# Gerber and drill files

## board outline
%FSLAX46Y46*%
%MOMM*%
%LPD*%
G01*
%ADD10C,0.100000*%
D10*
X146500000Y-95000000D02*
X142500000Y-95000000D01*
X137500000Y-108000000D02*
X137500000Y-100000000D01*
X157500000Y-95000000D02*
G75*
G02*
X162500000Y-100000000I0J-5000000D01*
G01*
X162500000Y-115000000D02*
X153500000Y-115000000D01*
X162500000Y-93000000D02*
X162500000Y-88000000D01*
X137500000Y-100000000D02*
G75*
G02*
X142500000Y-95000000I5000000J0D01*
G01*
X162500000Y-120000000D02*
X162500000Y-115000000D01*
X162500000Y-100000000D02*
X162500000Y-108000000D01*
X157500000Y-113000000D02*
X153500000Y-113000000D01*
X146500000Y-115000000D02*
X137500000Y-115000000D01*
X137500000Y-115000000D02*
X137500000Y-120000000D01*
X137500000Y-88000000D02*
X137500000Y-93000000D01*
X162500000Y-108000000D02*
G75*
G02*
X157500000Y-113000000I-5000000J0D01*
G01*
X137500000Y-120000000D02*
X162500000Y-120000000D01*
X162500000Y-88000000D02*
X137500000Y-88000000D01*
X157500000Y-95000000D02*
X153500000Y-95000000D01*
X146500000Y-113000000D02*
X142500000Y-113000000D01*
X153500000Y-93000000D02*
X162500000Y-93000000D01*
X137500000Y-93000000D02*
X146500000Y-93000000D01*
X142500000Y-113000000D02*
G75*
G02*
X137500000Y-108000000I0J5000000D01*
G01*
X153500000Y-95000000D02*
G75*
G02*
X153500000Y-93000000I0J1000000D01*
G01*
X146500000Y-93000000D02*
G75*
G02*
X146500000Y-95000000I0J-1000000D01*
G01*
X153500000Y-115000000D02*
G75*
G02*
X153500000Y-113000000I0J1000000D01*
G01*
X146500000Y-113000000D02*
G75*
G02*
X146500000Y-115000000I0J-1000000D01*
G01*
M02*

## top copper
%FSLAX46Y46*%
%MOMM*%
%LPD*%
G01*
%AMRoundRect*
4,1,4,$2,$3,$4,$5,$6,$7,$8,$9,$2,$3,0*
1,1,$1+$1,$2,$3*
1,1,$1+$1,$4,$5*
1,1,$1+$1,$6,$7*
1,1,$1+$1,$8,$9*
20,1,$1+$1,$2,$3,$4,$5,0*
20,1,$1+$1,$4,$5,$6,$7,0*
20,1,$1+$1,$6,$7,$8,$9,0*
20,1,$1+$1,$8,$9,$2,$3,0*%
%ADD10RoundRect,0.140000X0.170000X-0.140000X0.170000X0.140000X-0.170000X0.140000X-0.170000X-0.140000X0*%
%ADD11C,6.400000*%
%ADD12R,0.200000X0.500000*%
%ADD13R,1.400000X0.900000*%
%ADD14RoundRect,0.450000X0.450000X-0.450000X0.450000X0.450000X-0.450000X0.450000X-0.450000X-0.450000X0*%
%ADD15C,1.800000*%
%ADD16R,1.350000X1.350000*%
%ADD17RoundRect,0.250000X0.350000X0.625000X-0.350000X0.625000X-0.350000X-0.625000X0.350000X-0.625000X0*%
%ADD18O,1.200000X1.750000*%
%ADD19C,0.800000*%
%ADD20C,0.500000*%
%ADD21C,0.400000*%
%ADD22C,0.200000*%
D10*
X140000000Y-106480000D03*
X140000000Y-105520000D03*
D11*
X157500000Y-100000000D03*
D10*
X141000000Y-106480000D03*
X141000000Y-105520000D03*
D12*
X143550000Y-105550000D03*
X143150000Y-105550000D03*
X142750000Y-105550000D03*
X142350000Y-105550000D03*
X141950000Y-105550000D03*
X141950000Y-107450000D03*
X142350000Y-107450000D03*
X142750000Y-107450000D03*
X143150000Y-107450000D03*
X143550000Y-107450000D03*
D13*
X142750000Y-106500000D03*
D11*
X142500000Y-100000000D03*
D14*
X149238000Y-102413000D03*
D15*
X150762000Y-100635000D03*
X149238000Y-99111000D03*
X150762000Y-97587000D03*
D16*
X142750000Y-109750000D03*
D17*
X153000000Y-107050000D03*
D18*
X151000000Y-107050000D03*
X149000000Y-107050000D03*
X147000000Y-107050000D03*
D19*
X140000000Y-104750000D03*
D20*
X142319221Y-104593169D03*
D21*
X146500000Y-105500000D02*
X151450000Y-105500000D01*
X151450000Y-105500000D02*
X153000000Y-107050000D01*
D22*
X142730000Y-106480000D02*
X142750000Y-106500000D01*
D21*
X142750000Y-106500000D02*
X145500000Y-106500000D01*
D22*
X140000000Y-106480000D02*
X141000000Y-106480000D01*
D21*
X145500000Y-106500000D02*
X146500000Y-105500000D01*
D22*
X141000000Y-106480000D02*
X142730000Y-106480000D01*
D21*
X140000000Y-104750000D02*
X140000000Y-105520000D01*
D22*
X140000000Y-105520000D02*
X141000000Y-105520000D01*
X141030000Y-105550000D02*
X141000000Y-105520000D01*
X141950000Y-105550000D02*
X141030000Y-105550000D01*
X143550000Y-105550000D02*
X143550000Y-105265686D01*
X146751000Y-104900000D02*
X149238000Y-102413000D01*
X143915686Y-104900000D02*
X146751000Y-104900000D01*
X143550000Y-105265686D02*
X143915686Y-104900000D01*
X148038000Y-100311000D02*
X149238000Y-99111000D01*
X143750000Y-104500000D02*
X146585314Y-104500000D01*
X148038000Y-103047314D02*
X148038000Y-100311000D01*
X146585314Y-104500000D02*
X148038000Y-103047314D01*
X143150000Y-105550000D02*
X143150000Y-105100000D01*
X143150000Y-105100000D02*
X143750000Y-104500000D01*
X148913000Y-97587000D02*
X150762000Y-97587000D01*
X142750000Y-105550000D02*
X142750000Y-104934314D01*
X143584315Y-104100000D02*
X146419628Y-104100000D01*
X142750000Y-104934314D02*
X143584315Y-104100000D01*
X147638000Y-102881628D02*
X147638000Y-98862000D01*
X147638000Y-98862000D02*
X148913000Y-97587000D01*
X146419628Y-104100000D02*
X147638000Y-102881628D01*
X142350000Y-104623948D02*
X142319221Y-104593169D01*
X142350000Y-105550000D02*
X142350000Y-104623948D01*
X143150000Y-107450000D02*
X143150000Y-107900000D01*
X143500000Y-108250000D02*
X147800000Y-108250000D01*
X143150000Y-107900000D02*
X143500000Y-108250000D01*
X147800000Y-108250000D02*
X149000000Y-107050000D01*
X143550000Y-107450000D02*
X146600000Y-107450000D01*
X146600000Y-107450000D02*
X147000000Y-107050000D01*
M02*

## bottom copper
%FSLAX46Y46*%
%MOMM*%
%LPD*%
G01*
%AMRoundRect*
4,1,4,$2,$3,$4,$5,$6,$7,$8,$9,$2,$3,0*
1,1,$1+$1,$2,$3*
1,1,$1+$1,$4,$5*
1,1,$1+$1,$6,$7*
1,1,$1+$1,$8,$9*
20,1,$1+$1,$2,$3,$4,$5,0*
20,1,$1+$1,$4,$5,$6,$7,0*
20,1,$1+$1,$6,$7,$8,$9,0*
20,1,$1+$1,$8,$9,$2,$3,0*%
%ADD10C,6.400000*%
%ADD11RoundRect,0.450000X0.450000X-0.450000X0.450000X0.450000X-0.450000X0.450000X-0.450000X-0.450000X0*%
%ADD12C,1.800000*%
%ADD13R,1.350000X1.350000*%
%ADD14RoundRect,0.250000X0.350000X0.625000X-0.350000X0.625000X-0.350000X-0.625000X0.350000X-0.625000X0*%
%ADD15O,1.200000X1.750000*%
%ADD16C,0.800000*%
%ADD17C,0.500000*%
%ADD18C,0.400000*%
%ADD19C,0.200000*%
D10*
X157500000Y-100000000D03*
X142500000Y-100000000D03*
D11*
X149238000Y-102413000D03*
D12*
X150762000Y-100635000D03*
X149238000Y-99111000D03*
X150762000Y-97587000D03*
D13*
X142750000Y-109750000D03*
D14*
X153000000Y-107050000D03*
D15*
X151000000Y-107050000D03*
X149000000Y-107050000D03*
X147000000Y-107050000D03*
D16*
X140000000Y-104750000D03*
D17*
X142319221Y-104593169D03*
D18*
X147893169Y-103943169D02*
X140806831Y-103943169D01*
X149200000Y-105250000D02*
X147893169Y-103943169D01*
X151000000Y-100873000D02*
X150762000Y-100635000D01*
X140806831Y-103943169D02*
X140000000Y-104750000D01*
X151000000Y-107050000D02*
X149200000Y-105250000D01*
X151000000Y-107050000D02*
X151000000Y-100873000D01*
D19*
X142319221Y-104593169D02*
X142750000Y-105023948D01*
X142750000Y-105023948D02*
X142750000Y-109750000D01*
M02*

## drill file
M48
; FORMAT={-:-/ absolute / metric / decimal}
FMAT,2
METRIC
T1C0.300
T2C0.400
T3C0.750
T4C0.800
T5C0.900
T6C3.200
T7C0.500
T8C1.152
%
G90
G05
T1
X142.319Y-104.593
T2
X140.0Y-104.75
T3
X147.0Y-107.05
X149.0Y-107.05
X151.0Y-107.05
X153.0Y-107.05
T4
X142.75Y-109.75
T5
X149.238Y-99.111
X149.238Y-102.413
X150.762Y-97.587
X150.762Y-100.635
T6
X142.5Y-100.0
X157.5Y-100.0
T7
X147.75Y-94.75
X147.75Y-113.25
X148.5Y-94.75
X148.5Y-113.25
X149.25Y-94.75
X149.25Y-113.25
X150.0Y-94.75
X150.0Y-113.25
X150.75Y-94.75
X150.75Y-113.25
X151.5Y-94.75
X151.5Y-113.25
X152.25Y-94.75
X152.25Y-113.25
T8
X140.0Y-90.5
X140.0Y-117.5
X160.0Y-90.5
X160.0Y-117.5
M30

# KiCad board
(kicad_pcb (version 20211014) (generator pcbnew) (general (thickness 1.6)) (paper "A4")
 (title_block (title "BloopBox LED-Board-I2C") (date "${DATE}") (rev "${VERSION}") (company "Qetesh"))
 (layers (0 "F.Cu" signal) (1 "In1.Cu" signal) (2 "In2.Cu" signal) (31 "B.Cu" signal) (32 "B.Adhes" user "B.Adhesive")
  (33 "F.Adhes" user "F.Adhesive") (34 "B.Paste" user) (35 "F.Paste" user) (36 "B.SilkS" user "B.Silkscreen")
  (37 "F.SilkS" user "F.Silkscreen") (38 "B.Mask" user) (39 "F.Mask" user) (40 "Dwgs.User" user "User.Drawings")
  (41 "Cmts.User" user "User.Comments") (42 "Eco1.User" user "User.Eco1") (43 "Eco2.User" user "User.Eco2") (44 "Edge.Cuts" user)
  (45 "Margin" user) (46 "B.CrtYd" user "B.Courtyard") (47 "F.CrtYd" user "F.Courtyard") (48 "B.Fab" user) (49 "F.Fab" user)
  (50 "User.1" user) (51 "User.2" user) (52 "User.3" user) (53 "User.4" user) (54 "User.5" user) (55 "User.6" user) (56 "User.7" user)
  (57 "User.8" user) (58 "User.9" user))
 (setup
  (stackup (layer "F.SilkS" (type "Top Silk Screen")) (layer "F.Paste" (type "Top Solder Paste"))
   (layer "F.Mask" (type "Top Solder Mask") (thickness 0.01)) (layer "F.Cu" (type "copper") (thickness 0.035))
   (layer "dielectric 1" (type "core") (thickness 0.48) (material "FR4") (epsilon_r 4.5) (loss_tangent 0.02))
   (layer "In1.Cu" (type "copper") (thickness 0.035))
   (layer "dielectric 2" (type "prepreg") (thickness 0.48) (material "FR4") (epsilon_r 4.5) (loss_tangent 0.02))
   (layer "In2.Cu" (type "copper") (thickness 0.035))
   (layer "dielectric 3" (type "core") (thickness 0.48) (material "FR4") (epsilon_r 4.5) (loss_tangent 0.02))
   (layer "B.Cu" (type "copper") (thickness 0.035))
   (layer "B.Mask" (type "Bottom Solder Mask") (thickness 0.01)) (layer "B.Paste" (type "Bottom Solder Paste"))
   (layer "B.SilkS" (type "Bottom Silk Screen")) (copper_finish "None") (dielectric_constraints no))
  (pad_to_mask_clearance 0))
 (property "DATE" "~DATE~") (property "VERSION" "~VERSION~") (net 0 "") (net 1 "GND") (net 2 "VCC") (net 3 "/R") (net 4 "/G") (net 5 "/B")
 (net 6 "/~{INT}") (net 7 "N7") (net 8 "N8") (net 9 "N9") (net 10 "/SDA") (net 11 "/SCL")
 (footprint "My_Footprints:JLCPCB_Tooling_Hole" (layer "F.Cu") (at 160 90.5)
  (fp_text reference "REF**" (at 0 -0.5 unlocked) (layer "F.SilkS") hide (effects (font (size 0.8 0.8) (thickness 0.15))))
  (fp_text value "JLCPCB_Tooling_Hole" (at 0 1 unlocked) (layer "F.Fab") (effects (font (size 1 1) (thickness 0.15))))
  (pad "" np_thru_hole circle (at 0 0) (size 1.152 1.152) (drill 1.152) (layers F&B.Cu *.Mask) (solder_mask_margin 0.148) (clearance 0.248)))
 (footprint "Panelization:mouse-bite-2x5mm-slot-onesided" (layer "F.Cu") (at 150 94 180)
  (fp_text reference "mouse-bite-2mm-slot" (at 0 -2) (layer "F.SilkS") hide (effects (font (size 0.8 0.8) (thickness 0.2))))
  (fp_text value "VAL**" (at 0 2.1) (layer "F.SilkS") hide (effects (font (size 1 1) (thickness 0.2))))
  (fp_arc (start -3.5 -1) (mid -2.5 0) (end -3.5 1) (layer "Edge.Cuts") (width 0.1))
  (fp_arc (start 3.5 1) (mid 2.5 0) (end 3.5 -1) (layer "Edge.Cuts") (width 0.1))
  (pad "" np_thru_hole circle (at 1.5 -0.75 180) (size 0.5 0.5) (drill 0.5) (layers *.Cu *.Mask))
  (pad "" np_thru_hole circle (at -1.5 -0.75 180) (size 0.5 0.5) (drill 0.5) (layers *.Cu *.Mask))
  (pad "" np_thru_hole circle (at -0.75 -0.75 180) (size 0.5 0.5) (drill 0.5) (layers *.Cu *.Mask))
  (pad "" np_thru_hole circle (at 2.25 -0.75 180) (size 0.5 0.5) (drill 0.5) (layers *.Cu *.Mask))
  (pad "" np_thru_hole circle (at 0.75 -0.75 180) (size 0.5 0.5) (drill 0.5) (layers *.Cu *.Mask))
  (pad "" np_thru_hole circle (at -2.25 -0.75 180) (size 0.5 0.5) (drill 0.5) (layers *.Cu *.Mask))
  (pad "" np_thru_hole circle (at 0 -0.75 180) (size 0.5 0.5) (drill 0.5) (layers *.Cu *.Mask)))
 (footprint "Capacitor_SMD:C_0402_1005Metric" (layer "F.Cu") (at 140 106 90)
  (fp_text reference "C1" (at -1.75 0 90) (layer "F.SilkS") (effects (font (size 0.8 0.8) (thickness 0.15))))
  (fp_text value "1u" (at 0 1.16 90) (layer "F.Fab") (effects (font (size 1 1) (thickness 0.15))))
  (pad "1" smd roundrect (at -0.48 0 90) (size 0.56 0.62) (layers "F.Cu" "F.Paste" "F.Mask") (roundrect_rratio 0.25) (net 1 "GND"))
  (pad "2" smd roundrect (at 0.48 0 90) (size 0.56 0.62) (layers "F.Cu" "F.Paste" "F.Mask") (roundrect_rratio 0.25) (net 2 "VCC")))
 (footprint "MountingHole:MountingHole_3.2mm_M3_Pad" (layer "F.Cu") (at 157.5 100)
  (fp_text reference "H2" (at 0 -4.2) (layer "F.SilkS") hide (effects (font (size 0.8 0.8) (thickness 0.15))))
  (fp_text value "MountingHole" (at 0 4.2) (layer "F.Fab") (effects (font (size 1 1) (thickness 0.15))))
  (pad "" thru_hole circle (at 0 0) (size 6.4 6.4) (drill 3.2) (layers *.Cu *.Mask)))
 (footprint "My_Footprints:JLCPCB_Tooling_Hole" (layer "F.Cu") (at 140 90.5)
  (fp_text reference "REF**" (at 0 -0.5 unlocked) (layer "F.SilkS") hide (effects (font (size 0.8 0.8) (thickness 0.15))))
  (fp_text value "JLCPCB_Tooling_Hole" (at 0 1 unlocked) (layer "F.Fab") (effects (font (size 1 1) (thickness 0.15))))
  (pad "" np_thru_hole circle (at 0 0) (size 1.152 1.152) (drill 1.152) (layers F&B.Cu *.Mask) (solder_mask_margin 0.148) (clearance 0.248)))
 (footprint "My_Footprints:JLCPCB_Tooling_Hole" (layer "F.Cu") (at 140 117.5)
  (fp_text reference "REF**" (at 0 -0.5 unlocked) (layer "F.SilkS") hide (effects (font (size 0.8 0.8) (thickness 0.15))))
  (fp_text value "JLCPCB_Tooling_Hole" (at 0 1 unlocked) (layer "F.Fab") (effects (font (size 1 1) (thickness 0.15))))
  (pad "" np_thru_hole circle (at 0 0) (size 1.152 1.152) (drill 1.152) (layers F&B.Cu *.Mask) (solder_mask_margin 0.148) (clearance 0.248)))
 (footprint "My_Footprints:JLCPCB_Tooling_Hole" (layer "F.Cu") (at 160 117.5)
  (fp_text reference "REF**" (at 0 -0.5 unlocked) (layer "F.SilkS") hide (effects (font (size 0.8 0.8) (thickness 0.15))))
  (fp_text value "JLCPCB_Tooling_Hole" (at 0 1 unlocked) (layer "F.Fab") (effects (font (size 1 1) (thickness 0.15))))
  (pad "" np_thru_hole circle (at 0 0) (size 1.152 1.152) (drill 1.152) (layers F&B.Cu *.Mask) (solder_mask_margin 0.148) (clearance 0.248)))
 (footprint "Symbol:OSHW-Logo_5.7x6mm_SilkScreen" (layer "F.Cu") (at 158.8 108)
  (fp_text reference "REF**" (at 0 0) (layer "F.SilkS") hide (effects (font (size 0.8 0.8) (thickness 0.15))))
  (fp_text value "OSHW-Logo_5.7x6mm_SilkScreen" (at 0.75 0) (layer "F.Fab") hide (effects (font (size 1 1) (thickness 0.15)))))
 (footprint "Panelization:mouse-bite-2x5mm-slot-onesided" (layer "F.Cu") (at 150 114)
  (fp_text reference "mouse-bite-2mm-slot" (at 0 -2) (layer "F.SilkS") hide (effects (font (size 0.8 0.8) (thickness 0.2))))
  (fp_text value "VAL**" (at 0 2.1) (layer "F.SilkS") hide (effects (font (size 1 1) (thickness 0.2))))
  (fp_arc (start 3.5 1) (mid 2.5 0) (end 3.5 -1) (layer "Edge.Cuts") (width 0.1))
  (fp_arc (start -3.5 -1) (mid -2.5 0) (end -3.5 1) (layer "Edge.Cuts") (width 0.1))
  (pad "" np_thru_hole circle (at -1.5 -0.75) (size 0.5 0.5) (drill 0.5) (layers *.Cu *.Mask))
  (pad "" np_thru_hole circle (at 2.25 -0.75) (size 0.5 0.5) (drill 0.5) (layers *.Cu *.Mask))
  (pad "" np_thru_hole circle (at -2.25 -0.75) (size 0.5 0.5) (drill 0.5) (layers *.Cu *.Mask))
  (pad "" np_thru_hole circle (at 0.75 -0.75) (size 0.5 0.5) (drill 0.5) (layers *.Cu *.Mask))
  (pad "" np_thru_hole circle (at 0 -0.75) (size 0.5 0.5) (drill 0.5) (layers *.Cu *.Mask))
  (pad "" np_thru_hole circle (at 1.5 -0.75) (size 0.5 0.5) (drill 0.5) (layers *.Cu *.Mask))
  (pad "" np_thru_hole circle (at -0.75 -0.75) (size 0.5 0.5) (drill 0.5) (layers *.Cu *.Mask)))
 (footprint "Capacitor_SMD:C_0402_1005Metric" (layer "F.Cu") (at 141 106 90)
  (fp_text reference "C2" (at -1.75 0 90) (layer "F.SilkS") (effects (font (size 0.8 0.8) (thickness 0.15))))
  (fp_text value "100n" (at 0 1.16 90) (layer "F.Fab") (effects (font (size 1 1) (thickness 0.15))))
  (pad "1" smd roundrect (at -0.48 0 90) (size 0.56 0.62) (layers "F.Cu" "F.Paste" "F.Mask") (roundrect_rratio 0.25) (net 1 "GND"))
  (pad "2" smd roundrect (at 0.48 0 90) (size 0.56 0.62) (layers "F.Cu" "F.Paste" "F.Mask") (roundrect_rratio 0.25) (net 2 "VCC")))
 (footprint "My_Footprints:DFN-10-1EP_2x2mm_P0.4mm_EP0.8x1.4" (layer "F.Cu") (at 142.75 106.5 -90)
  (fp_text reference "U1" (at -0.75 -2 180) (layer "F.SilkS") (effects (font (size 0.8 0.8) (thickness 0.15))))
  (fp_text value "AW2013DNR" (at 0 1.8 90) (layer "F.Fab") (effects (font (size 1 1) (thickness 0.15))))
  (pad "1" smd rect (at -0.95 -0.8 270) (size 0.5 0.2) (layers "F.Cu" "F.Paste" "F.Mask") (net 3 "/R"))
  (pad "2" smd rect (at -0.95 -0.4 270) (size 0.5 0.2) (layers "F.Cu" "F.Paste" "F.Mask") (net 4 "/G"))
  (pad "3" smd rect (at -0.95 0 270) (size 0.5 0.2) (layers "F.Cu" "F.Paste" "F.Mask") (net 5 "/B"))
  (pad "4" smd rect (at -0.95 0.4 270) (size 0.5 0.2) (layers "F.Cu" "F.Paste" "F.Mask") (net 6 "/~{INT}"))
  (pad "5" smd rect (at -0.95 0.8 270) (size 0.5 0.2) (layers "F.Cu" "F.Paste" "F.Mask") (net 2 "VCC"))
  (pad "6" smd rect (at 0.95 0.8 270) (size 0.5 0.2) (layers "F.Cu" "F.Paste" "F.Mask") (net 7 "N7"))
  (pad "7" smd rect (at 0.95 0.4 270) (size 0.5 0.2) (layers "F.Cu" "F.Paste" "F.Mask") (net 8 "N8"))
  (pad "8" smd rect (at 0.95 0 270) (size 0.5 0.2) (layers "F.Cu" "F.Paste" "F.Mask") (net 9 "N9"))
  (pad "9" smd rect (at 0.95 -0.4 270) (size 0.5 0.2) (layers "F.Cu" "F.Paste" "F.Mask") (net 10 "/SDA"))
  (pad "10" smd rect (at 0.95 -0.8 270) (size 0.5 0.2) (layers "F.Cu" "F.Paste" "F.Mask") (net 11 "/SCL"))
  (pad "11" smd rect (at 0 0 270) (size 0.9 1.4) (layers "F.Cu" "F.Paste" "F.Mask") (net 1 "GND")))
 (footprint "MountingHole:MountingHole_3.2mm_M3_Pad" (layer "F.Cu") (at 142.5 100)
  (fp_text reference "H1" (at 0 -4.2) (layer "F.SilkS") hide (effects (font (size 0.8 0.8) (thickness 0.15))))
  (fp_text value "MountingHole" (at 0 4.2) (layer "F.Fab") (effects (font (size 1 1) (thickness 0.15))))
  (pad "" thru_hole circle (at 0 0) (size 6.4 6.4) (drill 3.2) (layers *.Cu *.Mask)))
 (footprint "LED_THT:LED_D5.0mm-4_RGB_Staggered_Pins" (layer "F.Cu") (at 150 100 90)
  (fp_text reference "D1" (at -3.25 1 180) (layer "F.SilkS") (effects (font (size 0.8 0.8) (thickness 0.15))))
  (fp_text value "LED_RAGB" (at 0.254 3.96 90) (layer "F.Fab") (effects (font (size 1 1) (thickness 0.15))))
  (pad "1" thru_hole roundrect (at -2.413 -0.762 90) (size 1.8 1.8) (drill 0.9) (layers *.Cu *.Mask) (roundrect_rratio 0.25) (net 3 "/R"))
  (pad "2" thru_hole circle (at -0.635 0.762 90) (size 1.8 1.8) (drill 0.9) (layers *.Cu *.Mask) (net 2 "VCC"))
  (pad "3" thru_hole circle (at 0.889 -0.762 90) (size 1.8 1.8) (drill 0.9) (layers *.Cu *.Mask) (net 4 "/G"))
  (pad "4" thru_hole circle (at 2.413 0.762 90) (size 1.8 1.8) (drill 0.9) (layers *.Cu *.Mask) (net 5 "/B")))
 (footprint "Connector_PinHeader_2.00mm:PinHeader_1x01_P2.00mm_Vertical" (layer "B.Cu") (at 142.75 109.75 180)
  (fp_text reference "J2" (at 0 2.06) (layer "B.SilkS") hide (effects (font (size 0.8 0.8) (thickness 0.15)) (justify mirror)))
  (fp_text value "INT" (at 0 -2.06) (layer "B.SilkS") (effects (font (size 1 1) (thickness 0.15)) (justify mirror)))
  (pad "1" thru_hole rect (at 0 0 180) (size 1.35 1.35) (drill 0.8) (layers *.Cu *.Mask) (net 6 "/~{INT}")))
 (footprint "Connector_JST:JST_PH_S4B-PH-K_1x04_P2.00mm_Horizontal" (layer "B.Cu") (at 153 107.05 180)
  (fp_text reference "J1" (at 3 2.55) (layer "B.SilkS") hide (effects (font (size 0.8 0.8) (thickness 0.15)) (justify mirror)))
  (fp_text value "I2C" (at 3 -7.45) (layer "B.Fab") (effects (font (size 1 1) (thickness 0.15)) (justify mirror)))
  (pad "1" thru_hole roundrect (at 0 0 180) (size 1.2 1.75) (drill 0.75) (layers *.Cu *.Mask) (roundrect_rratio 0.2083333333) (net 1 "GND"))
  (pad "2" thru_hole oval (at 2 0 180) (size 1.2 1.75) (drill 0.75) (layers *.Cu *.Mask) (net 2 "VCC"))
  (pad "3" thru_hole oval (at 4 0 180) (size 1.2 1.75) (drill 0.75) (layers *.Cu *.Mask) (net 10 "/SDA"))
  (pad "4" thru_hole oval (at 6 0 180) (size 1.2 1.75) (drill 0.75) (layers *.Cu *.Mask) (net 11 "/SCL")))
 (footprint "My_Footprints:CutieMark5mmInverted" (layer "B.Cu") (at 158.5 107 180)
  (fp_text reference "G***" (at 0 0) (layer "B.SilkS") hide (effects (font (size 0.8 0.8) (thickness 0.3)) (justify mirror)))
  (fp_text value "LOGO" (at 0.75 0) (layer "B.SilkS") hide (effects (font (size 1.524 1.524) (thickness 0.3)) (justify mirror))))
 (gr_line (start 146.5 95) (end 142.5 95) (layer "Edge.Cuts") (width 0.1))
 (gr_line (start 137.5 108) (end 137.5 100) (layer "Edge.Cuts") (width 0.1))
 (gr_arc (start 157.5 95) (mid 161.035534 96.464466) (end 162.5 100) (layer "Edge.Cuts") (width 0.1))
 (gr_line (start 162.5 115) (end 153.5 115) (layer "Edge.Cuts") (width 0.1))
 (gr_line (start 162.5 93) (end 162.5 88) (layer "Edge.Cuts") (width 0.1))
 (gr_arc (start 137.5 100) (mid 138.964466 96.464466) (end 142.5 95) (layer "Edge.Cuts") (width 0.1))
 (gr_line (start 162.5 120) (end 162.5 115) (layer "Edge.Cuts") (width 0.1))
 (gr_line (start 162.5 100) (end 162.5 108) (layer "Edge.Cuts") (width 0.1))
 (gr_line (start 157.5 113) (end 153.5 113) (layer "Edge.Cuts") (width 0.1))
 (gr_line (start 146.5 115) (end 137.5 115) (layer "Edge.Cuts") (width 0.1))
 (gr_line (start 137.5 115) (end 137.5 120) (layer "Edge.Cuts") (width 0.1))
 (gr_line (start 137.5 88) (end 137.5 93) (layer "Edge.Cuts") (width 0.1))
 (gr_arc (start 162.5 108) (mid 161.035534 111.535534) (end 157.5 113) (layer "Edge.Cuts") (width 0.1))
 (gr_line (start 137.5 120) (end 162.5 120) (layer "Edge.Cuts") (width 0.1))
 (gr_line (start 162.5 88) (end 137.5 88) (layer "Edge.Cuts") (width 0.1))
 (gr_line (start 157.5 95) (end 153.5 95) (layer "Edge.Cuts") (width 0.1))
 (gr_line (start 146.5 113) (end 142.5 113) (layer "Edge.Cuts") (width 0.1))
 (gr_line (start 153.5 93) (end 162.5 93) (layer "Edge.Cuts") (width 0.1))
 (gr_line (start 137.5 93) (end 146.5 93) (layer "Edge.Cuts") (width 0.1))
 (gr_arc (start 142.5 113) (mid 138.964466 111.535534) (end 137.5 108) (layer "Edge.Cuts") (width 0.1))
 (segment (start 146.5 105.5) (end 151.45 105.5) (width 0.4) (layer "F.Cu") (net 1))
 (segment (start 151.45 105.5) (end 153 107.05) (width 0.4) (layer "F.Cu") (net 1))
 (segment (start 142.73 106.48) (end 142.75 106.5) (width 0.2) (layer "F.Cu") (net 1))
 (segment (start 142.75 106.5) (end 145.5 106.5) (width 0.4) (layer "F.Cu") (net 1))
 (segment (start 140 106.48) (end 141 106.48) (width 0.2) (layer "F.Cu") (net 1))
 (segment (start 145.5 106.5) (end 146.5 105.5) (width 0.4) (layer "F.Cu") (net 1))
 (segment (start 141 106.48) (end 142.73 106.48) (width 0.2) (layer "F.Cu") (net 1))
 (segment (start 140 104.75) (end 140 105.52) (width 0.4) (layer "F.Cu") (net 2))
 (segment (start 140 105.52) (end 141 105.52) (width 0.2) (layer "F.Cu") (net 2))
 (segment (start 141.03 105.55) (end 141 105.52) (width 0.2) (layer "F.Cu") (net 2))
 (segment (start 141.95 105.55) (end 141.03 105.55) (width 0.2) (layer "F.Cu") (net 2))
 (via (at 140 104.75) (size 0.8) (drill 0.4) (layers "F.Cu" "B.Cu") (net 2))
 (segment (start 147.893169 103.943169) (end 140.806831 103.943169) (width 0.4) (layer "B.Cu") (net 2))
 (segment (start 149.2 105.25) (end 147.893169 103.943169) (width 0.4) (layer "B.Cu") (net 2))
 (segment (start 151 100.873) (end 150.762 100.635) (width 0.4) (layer "B.Cu") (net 2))
 (segment (start 140.806831 103.943169) (end 140 104.75) (width 0.4) (layer "B.Cu") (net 2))
 (segment (start 151 107.05) (end 149.2 105.25) (width 0.4) (layer "B.Cu") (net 2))
 (segment (start 151 107.05) (end 151 100.873) (width 0.4) (layer "B.Cu") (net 2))
 (segment (start 143.55 105.55) (end 143.55 105.265686) (width 0.2) (layer "F.Cu") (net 3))
 (segment (start 146.751 104.9) (end 149.238 102.413) (width 0.2) (layer "F.Cu") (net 3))
 (segment (start 143.915686 104.9) (end 146.751 104.9) (width 0.2) (layer "F.Cu") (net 3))
 (segment (start 143.55 105.265686) (end 143.915686 104.9) (width 0.2) (layer "F.Cu") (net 3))
 (segment (start 148.038 100.311) (end 149.238 99.111) (width 0.2) (layer "F.Cu") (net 4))
 (segment (start 143.75 104.5) (end 146.585314 104.5) (width 0.2) (layer "F.Cu") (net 4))
 (segment (start 148.038 103.047314) (end 148.038 100.311) (width 0.2) (layer "F.Cu") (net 4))
 (segment (start 146.585314 104.5) (end 148.038 103.047314) (width 0.2) (layer "F.Cu") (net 4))
 (segment (start 143.15 105.55) (end 143.15 105.1) (width 0.2) (layer "F.Cu") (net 4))
 (segment (start 143.15 105.1) (end 143.75 104.5) (width 0.2) (layer "F.Cu") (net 4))
 (segment (start 148.913 97.587) (end 150.762 97.587) (width 0.2) (layer "F.Cu") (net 5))
 (segment (start 142.75 105.55) (end 142.75 104.934314) (width 0.2) (layer "F.Cu") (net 5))
 (segment (start 143.584315 104.1) (end 146.419628 104.1) (width 0.2) (layer "F.Cu") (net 5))
 (segment (start 142.75 104.934314) (end 143.584315 104.1) (width 0.2) (layer "F.Cu") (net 5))
 (segment (start 147.638 102.881628) (end 147.638 98.862) (width 0.2) (layer "F.Cu") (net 5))
 (segment (start 147.638 98.862) (end 148.913 97.587) (width 0.2) (layer "F.Cu") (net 5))
 (segment (start 146.419628 104.1) (end 147.638 102.881628) (width 0.2) (layer "F.Cu") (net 5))
 (segment (start 142.35 104.623948) (end 142.319221 104.593169) (width 0.2) (layer "F.Cu") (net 6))
 (segment (start 142.35 105.55) (end 142.35 104.623948) (width 0.2) (layer "F.Cu") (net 6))
 (via (at 142.319221 104.593169) (size 0.5) (drill 0.3) (layers "F.Cu" "B.Cu") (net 6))
 (segment (start 142.319221 104.593169) (end 142.75 105.023948) (width 0.2) (layer "B.Cu") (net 6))
 (segment (start 142.75 105.023948) (end 142.75 109.75) (width 0.2) (layer "B.Cu") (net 6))
 (segment (start 143.15 107.45) (end 143.15 107.9) (width 0.2) (layer "F.Cu") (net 10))
 (segment (start 143.5 108.25) (end 147.8 108.25) (width 0.2) (layer "F.Cu") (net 10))
 (segment (start 143.15 107.9) (end 143.5 108.25) (width 0.2) (layer "F.Cu") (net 10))
 (segment (start 147.8 108.25) (end 149 107.05) (width 0.2) (layer "F.Cu") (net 10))
 (segment (start 143.55 107.45) (end 146.6 107.45) (width 0.2) (layer "F.Cu") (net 11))
 (segment (start 146.6 107.45) (end 147 107.05) (width 0.2) (layer "F.Cu") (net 11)))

